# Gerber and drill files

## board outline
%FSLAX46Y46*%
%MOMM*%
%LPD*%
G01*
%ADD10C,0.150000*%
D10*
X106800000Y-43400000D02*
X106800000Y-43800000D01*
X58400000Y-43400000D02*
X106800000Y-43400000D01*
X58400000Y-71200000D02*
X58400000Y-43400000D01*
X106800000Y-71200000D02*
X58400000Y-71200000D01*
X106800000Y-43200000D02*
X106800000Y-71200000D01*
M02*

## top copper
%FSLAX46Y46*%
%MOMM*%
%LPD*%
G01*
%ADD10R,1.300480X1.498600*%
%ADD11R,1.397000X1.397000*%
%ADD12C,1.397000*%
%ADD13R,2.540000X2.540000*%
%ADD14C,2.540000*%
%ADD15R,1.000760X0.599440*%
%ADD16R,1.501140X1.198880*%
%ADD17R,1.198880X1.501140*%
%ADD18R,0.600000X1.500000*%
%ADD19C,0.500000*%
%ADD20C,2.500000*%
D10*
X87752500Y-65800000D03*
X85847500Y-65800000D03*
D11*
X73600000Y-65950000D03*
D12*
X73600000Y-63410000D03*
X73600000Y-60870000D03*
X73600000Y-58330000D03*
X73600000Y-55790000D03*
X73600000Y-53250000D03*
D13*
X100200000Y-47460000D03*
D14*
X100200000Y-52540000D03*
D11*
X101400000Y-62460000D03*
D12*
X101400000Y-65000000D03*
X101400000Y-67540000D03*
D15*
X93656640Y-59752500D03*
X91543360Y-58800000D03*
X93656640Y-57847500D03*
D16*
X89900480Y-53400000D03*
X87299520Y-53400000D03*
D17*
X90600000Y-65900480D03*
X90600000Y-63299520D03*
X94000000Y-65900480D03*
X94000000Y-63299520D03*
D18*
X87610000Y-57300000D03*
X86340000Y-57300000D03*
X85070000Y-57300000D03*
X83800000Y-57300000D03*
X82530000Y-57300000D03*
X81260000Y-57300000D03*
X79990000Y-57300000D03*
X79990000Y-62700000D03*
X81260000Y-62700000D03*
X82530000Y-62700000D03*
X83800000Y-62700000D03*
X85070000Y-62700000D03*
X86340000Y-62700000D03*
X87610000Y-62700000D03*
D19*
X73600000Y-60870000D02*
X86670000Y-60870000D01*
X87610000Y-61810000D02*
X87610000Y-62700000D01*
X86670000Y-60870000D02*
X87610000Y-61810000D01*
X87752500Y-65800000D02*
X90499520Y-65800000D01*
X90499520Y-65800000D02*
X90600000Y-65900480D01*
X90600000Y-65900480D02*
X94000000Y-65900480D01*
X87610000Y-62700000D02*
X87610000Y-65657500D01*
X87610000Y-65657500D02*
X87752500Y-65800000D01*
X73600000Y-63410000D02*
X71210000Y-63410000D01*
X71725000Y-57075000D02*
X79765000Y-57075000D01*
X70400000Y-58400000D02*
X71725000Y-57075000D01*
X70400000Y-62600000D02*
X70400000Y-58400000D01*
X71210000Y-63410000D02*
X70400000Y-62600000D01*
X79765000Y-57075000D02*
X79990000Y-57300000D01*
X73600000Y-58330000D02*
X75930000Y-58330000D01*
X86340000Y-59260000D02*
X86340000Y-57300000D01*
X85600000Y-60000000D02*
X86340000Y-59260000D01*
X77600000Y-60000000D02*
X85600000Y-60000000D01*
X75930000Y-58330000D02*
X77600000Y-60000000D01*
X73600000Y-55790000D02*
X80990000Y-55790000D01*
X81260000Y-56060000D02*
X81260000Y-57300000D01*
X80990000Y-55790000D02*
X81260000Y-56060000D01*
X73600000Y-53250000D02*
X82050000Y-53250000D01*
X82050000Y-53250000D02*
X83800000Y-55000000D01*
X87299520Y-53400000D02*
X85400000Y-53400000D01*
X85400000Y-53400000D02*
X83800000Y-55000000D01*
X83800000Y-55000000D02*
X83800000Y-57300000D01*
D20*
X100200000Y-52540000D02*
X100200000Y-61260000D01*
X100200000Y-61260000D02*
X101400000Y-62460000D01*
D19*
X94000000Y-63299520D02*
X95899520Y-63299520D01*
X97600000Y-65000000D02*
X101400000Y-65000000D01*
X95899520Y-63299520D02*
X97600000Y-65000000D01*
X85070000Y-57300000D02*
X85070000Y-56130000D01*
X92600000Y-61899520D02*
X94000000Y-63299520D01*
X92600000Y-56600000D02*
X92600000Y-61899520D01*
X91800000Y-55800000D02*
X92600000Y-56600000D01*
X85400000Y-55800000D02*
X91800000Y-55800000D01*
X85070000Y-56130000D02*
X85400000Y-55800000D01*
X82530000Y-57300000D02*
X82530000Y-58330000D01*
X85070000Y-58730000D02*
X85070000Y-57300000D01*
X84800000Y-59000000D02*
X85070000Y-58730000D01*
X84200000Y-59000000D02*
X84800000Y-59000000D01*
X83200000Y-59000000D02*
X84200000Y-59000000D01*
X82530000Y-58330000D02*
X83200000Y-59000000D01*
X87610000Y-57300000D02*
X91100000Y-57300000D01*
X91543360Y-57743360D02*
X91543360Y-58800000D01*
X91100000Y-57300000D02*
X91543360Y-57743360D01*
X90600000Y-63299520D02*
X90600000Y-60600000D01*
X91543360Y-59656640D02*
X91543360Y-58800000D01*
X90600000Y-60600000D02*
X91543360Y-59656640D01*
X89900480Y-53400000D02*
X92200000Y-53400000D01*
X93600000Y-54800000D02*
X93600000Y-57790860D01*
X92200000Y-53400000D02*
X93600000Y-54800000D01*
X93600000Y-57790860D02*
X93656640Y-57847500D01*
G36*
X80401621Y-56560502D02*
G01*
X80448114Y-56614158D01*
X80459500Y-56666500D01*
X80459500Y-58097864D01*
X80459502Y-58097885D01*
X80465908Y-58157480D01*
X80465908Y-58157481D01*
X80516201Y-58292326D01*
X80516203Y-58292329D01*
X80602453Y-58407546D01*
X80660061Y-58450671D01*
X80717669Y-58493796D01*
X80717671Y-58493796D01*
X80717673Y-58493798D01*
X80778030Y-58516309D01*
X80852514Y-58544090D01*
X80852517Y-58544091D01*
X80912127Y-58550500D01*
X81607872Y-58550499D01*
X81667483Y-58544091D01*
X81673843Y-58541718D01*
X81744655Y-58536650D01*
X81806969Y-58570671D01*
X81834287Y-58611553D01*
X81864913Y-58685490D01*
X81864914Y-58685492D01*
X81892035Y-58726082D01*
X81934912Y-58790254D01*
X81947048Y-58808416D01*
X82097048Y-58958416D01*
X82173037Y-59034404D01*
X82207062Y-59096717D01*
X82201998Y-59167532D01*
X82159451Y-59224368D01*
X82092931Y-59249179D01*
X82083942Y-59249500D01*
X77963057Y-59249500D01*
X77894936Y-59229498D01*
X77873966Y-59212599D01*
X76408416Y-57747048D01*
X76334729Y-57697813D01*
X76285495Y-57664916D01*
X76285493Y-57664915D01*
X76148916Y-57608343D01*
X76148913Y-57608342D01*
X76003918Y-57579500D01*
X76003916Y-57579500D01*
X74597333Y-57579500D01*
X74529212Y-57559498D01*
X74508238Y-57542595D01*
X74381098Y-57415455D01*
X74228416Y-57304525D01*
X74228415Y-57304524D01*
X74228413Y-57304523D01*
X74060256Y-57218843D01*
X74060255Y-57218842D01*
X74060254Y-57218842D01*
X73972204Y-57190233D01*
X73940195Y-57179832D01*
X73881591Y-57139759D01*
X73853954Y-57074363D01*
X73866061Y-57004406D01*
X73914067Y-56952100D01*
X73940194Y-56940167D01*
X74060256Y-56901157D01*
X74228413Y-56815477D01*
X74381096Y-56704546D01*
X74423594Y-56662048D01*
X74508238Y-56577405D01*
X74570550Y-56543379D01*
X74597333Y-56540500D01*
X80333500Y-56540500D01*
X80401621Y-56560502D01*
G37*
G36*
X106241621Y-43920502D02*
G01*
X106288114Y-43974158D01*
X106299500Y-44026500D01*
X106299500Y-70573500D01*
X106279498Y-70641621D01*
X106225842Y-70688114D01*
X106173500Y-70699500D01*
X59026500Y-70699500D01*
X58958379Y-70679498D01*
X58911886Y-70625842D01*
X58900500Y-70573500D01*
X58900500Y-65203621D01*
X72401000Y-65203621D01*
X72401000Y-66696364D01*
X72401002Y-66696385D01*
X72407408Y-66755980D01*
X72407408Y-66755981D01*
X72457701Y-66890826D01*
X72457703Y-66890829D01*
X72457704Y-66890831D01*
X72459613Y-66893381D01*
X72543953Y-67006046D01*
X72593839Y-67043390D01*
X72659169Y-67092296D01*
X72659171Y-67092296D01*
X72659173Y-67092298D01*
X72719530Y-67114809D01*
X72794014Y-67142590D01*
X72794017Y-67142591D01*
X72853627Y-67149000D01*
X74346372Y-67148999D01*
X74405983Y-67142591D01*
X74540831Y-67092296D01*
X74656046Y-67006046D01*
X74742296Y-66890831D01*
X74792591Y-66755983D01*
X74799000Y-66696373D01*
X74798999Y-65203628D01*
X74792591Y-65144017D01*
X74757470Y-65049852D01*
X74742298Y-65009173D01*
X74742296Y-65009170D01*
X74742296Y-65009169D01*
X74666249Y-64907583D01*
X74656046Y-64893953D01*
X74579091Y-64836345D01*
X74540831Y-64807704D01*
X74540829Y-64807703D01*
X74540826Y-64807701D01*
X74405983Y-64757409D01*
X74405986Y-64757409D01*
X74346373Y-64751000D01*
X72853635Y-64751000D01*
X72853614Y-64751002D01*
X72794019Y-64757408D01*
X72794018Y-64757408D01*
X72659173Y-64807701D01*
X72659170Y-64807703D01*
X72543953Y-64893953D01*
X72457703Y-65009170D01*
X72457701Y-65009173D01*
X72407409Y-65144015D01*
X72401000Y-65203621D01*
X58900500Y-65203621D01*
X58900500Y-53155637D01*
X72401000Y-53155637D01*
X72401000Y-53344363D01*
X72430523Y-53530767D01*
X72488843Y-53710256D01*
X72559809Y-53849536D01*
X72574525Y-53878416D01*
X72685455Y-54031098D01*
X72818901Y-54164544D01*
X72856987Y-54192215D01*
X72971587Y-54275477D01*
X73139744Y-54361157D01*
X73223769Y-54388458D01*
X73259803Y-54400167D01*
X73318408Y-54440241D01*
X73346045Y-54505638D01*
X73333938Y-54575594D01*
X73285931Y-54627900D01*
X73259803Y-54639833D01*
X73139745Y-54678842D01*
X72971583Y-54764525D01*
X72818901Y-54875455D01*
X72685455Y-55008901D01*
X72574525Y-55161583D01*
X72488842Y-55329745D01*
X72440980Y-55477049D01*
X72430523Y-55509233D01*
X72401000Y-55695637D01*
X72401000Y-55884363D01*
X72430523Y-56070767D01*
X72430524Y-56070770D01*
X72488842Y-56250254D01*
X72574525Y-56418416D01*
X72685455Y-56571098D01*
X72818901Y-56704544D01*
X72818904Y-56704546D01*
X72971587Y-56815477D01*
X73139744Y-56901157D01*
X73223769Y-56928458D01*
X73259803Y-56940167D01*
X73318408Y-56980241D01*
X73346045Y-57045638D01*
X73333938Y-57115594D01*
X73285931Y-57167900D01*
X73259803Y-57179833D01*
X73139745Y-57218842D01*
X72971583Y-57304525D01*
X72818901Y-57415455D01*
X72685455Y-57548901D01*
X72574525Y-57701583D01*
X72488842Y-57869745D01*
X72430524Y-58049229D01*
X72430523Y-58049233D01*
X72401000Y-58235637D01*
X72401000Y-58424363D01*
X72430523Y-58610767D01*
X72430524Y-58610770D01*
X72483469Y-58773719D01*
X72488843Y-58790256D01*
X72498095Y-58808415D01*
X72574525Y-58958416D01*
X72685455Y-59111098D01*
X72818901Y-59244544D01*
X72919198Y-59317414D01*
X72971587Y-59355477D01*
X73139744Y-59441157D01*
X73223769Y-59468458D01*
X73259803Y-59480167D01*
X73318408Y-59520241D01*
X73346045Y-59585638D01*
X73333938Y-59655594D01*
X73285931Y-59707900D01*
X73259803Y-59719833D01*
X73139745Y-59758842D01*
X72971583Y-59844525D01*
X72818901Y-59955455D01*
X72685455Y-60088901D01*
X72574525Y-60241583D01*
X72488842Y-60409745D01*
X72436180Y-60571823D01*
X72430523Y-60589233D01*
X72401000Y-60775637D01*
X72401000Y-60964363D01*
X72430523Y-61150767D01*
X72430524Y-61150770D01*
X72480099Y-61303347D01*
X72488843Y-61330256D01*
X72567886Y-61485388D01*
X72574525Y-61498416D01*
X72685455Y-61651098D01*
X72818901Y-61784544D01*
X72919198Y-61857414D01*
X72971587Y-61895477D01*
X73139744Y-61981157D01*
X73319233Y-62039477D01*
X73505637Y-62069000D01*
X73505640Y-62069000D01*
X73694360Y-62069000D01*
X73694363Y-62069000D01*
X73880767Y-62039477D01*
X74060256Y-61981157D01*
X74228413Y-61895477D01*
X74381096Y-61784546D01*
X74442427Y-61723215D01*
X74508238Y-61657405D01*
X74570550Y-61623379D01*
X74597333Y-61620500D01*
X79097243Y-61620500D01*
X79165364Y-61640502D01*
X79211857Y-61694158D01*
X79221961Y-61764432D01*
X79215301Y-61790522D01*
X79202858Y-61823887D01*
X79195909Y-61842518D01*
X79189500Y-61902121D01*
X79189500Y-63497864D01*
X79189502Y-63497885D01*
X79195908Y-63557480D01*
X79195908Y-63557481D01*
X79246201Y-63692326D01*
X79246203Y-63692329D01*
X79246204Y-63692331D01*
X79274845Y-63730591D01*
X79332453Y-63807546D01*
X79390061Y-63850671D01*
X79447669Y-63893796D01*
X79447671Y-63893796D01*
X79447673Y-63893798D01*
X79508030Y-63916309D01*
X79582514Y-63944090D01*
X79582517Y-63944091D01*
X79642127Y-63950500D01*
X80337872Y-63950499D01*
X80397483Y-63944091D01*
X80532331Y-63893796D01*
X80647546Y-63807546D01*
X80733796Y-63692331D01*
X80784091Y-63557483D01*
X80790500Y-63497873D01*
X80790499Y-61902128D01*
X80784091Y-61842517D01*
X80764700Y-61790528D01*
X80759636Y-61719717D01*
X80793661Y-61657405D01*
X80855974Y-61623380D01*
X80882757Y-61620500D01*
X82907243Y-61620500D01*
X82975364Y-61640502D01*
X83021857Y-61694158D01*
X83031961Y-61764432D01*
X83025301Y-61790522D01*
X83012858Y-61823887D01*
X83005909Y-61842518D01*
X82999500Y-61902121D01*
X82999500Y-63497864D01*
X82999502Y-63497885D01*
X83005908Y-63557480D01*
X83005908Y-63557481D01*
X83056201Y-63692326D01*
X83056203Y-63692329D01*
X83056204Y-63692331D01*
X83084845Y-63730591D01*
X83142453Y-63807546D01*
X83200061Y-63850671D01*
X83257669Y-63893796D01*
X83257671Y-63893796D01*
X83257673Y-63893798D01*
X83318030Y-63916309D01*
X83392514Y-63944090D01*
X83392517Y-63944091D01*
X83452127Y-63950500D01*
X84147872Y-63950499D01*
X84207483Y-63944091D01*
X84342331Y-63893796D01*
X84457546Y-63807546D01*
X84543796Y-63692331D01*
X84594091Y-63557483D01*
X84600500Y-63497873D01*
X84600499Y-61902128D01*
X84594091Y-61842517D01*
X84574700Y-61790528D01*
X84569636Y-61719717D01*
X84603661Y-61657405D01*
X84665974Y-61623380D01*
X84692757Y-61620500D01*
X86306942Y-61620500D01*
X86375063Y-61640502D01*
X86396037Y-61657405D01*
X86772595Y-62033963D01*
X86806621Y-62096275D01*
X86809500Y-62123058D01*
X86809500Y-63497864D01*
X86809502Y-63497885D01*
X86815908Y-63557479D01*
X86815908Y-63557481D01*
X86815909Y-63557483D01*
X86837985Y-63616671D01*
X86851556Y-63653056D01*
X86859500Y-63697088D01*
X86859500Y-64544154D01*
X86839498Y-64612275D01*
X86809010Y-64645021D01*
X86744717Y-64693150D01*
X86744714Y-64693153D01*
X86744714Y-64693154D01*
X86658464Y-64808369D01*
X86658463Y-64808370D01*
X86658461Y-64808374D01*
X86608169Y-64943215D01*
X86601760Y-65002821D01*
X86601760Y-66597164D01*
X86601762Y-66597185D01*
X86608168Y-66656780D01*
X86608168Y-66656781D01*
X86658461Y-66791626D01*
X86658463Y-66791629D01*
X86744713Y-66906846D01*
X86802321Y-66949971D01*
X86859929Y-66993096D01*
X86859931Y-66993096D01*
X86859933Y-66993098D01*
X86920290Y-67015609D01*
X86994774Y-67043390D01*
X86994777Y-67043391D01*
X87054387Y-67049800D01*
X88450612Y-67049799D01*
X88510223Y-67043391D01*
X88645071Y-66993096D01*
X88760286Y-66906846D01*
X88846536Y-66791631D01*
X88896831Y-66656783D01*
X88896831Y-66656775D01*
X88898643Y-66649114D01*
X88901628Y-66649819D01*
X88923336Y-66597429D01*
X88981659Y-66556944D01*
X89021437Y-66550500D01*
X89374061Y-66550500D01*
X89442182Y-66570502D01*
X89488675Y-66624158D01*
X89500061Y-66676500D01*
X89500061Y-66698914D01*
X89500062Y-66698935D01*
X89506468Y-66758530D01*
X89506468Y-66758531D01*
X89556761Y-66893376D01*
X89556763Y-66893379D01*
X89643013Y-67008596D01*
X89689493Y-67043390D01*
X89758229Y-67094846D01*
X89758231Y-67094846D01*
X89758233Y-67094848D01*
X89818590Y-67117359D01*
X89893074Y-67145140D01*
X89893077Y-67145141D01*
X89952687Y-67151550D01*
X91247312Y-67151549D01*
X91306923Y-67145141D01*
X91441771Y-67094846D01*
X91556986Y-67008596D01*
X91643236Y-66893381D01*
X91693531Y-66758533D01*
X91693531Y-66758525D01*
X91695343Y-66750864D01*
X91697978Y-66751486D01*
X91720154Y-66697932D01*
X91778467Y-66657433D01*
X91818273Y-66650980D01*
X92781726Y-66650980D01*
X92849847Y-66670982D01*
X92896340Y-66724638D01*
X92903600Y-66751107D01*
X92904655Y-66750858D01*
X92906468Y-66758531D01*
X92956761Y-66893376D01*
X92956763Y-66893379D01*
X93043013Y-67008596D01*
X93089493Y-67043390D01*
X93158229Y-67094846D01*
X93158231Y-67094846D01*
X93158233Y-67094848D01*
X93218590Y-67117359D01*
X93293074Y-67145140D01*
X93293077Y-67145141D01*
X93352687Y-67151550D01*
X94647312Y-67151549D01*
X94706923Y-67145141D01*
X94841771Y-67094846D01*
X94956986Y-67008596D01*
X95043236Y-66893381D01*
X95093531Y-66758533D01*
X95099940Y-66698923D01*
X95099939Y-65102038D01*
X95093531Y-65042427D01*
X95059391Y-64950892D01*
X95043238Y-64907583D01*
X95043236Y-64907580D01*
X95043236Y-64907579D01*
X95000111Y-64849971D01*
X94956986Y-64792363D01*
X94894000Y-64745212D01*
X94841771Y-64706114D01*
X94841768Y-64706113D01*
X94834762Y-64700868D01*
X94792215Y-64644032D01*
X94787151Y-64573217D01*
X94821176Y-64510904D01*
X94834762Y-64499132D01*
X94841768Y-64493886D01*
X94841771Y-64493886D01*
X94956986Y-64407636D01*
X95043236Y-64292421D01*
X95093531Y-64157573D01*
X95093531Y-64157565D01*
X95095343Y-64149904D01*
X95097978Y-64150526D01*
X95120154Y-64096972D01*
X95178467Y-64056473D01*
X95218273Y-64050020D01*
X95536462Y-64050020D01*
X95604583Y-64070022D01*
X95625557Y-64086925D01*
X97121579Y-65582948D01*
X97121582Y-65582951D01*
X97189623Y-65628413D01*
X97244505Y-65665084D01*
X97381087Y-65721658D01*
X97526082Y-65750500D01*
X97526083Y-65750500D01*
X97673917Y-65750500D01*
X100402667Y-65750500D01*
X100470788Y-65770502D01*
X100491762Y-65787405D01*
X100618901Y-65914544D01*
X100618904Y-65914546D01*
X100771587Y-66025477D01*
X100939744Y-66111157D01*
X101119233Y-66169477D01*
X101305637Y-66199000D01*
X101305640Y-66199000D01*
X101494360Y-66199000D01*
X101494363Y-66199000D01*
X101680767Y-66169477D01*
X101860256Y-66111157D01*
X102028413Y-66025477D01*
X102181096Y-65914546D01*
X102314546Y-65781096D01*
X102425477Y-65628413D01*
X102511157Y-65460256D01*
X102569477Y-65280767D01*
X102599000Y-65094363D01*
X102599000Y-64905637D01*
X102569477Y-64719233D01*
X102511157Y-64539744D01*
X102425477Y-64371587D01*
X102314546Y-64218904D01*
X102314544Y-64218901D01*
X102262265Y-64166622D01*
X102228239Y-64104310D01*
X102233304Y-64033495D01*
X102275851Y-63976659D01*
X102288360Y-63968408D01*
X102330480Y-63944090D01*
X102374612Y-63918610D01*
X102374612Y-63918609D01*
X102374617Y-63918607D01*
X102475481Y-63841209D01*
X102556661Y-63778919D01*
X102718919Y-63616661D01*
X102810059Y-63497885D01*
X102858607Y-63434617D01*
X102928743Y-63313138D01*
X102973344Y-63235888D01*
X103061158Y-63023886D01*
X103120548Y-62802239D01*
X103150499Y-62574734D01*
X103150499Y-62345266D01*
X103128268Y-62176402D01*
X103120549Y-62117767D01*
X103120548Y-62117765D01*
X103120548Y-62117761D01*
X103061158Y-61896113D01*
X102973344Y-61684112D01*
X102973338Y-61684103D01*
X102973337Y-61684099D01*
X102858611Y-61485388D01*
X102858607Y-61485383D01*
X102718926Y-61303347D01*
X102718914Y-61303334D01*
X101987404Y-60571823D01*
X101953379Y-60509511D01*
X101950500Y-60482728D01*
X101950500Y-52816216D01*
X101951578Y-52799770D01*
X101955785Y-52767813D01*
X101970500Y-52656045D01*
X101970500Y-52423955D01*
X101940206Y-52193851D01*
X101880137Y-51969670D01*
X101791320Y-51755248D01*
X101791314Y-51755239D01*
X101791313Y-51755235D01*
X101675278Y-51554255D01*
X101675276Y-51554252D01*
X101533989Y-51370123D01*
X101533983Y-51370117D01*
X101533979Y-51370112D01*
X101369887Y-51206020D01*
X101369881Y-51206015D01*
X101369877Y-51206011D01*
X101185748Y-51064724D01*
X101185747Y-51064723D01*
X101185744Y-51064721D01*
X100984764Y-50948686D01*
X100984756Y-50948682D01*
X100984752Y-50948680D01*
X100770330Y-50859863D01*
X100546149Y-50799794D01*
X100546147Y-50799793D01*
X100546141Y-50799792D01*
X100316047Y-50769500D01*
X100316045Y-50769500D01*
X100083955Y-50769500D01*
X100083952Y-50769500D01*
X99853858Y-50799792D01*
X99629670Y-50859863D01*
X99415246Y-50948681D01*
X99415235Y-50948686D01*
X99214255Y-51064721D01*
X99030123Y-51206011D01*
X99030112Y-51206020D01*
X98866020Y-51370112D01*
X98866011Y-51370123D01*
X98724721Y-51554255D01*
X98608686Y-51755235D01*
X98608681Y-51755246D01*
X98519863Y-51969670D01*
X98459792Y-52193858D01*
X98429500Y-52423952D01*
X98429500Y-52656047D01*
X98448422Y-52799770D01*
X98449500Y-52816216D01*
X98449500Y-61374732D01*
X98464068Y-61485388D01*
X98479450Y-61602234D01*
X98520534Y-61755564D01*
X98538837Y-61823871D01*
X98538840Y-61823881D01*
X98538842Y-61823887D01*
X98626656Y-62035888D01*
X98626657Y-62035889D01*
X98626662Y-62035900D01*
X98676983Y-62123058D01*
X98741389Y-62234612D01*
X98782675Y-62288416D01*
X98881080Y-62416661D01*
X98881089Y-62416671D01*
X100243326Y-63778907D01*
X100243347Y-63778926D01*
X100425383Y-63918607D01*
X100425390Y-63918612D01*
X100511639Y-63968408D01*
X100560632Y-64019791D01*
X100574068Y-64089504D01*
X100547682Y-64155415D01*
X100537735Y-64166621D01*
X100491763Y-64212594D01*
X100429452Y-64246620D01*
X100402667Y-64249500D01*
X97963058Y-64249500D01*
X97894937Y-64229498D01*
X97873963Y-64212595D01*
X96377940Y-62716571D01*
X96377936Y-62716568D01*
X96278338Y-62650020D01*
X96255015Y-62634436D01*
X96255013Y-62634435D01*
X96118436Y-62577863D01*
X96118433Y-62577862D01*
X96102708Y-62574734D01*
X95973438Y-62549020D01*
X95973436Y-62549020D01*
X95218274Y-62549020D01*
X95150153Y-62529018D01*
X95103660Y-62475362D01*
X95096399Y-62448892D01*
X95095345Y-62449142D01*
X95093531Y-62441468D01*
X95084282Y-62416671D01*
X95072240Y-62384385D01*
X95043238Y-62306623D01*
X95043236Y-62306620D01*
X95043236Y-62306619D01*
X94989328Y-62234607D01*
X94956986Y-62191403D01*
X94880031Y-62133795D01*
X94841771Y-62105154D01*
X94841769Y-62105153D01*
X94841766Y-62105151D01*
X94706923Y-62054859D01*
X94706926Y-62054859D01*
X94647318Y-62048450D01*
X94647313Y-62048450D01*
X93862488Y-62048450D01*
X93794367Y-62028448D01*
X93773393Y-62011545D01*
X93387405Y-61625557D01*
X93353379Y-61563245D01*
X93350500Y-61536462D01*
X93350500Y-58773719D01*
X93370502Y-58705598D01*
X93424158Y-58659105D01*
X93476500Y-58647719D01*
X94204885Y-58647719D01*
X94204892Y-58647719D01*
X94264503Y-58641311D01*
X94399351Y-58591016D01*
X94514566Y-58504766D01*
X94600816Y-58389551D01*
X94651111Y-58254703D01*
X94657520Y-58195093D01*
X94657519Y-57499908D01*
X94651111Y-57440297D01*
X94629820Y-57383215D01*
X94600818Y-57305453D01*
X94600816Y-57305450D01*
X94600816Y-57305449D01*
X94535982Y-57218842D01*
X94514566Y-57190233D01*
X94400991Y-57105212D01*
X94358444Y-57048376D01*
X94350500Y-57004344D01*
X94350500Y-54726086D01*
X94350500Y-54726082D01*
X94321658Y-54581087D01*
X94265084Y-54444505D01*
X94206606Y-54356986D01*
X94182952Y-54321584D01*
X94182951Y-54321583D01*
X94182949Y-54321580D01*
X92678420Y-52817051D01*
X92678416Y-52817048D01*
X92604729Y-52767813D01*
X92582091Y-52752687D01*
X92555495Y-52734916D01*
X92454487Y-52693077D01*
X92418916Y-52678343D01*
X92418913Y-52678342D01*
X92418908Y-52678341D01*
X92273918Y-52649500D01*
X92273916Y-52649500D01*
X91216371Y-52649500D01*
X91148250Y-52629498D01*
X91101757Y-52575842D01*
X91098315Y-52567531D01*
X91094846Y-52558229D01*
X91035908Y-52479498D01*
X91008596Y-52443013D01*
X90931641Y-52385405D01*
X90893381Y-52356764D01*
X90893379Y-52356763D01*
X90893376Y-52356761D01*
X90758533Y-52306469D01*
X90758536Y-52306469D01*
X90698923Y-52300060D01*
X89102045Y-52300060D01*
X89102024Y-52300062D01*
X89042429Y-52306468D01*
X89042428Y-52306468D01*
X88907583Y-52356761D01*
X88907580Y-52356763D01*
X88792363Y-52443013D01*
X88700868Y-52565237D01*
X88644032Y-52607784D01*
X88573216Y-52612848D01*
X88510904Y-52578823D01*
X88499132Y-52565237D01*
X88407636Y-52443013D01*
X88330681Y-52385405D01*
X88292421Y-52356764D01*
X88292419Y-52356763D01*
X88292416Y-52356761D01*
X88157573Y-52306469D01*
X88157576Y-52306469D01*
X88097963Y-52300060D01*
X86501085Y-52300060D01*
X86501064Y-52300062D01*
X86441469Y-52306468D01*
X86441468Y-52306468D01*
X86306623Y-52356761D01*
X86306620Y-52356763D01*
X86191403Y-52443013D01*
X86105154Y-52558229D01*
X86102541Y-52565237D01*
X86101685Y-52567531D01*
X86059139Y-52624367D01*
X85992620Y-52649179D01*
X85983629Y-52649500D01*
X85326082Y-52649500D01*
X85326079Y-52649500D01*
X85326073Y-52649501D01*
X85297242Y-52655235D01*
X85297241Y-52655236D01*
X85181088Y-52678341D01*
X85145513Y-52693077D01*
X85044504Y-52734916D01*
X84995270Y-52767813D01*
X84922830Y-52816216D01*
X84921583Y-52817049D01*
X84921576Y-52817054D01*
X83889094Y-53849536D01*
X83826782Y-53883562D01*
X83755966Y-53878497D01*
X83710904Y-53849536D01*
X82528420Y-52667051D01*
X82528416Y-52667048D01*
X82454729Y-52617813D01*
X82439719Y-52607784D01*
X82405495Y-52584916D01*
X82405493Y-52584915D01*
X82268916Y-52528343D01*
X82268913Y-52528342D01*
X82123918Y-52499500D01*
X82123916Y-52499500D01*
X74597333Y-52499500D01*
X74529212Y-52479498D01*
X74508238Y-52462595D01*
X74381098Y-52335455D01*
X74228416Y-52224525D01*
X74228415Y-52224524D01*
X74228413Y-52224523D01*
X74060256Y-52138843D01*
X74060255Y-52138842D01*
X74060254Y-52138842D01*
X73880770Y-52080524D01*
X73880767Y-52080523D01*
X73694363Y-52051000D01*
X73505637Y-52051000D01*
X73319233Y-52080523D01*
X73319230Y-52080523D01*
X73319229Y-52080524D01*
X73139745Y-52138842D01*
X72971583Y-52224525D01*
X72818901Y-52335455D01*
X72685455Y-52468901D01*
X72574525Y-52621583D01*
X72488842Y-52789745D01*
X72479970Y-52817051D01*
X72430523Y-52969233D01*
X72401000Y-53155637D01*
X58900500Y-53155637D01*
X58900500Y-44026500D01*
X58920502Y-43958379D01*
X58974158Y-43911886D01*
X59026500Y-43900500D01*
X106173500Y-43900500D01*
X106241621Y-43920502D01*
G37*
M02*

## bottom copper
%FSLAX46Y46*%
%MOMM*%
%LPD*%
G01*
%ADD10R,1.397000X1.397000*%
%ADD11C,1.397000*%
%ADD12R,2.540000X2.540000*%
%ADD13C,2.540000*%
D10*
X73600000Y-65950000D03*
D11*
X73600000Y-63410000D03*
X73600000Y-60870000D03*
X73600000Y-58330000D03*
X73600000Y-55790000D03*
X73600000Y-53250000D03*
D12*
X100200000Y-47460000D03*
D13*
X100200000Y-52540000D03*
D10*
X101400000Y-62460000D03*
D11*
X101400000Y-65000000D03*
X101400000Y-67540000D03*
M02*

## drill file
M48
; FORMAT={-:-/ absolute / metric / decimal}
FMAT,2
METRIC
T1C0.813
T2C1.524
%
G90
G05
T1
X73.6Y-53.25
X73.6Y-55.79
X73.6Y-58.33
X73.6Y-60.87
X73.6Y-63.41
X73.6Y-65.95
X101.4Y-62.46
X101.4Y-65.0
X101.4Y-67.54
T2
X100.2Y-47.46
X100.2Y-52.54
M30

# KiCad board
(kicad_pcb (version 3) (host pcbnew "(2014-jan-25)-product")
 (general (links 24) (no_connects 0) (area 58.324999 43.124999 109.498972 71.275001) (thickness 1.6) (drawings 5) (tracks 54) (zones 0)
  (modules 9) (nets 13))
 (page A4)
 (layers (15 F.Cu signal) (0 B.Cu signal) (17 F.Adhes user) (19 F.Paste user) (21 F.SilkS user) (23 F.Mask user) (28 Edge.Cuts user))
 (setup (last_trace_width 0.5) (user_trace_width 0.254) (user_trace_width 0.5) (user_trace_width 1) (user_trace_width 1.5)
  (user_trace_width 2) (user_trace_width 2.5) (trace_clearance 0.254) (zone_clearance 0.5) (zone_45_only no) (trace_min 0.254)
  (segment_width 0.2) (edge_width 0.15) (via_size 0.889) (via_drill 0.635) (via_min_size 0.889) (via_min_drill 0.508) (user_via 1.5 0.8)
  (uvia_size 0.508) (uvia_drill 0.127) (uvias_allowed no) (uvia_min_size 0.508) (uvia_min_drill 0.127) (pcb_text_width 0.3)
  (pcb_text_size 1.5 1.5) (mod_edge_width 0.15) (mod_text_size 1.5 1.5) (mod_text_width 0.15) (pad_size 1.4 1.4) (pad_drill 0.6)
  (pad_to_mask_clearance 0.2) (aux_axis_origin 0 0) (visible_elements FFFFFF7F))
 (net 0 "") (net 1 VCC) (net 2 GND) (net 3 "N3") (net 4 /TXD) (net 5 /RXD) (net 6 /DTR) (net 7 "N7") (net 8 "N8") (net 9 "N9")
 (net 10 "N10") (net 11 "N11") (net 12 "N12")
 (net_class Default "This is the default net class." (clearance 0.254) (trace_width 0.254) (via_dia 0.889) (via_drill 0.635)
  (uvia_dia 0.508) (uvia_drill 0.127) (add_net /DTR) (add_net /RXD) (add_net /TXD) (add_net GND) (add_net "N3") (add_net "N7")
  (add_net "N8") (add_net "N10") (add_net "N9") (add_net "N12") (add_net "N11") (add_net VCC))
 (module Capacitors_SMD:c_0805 (layer F.Cu) (at 86.8 65.8)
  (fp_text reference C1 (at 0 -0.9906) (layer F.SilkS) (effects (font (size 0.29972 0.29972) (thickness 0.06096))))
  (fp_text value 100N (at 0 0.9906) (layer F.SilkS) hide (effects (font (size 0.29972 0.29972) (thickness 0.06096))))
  (pad 1 smd rect (at 0.9525 0) (size 1.30048 1.4986) (layers F.Cu F.Paste F.Mask) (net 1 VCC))
  (pad 2 smd rect (at -0.9525 0) (size 1.30048 1.4986) (layers F.Cu F.Paste F.Mask) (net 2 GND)))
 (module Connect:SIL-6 (layer F.Cu) (at 73.6 59.6 90)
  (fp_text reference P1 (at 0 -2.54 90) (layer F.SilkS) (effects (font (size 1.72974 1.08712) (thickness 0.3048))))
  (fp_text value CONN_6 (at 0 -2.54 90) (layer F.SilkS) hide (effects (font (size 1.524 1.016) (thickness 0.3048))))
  (pad 1 thru_hole rect (at -6.35 0 90) (size 1.397 1.397) (drill 0.8128) (layers *.Cu *.Mask F.SilkS) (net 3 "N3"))
  (pad 2 thru_hole circle (at -3.81 0 90) (size 1.397 1.397) (drill 0.8128) (layers *.Cu *.Mask F.SilkS) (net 2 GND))
  (pad 3 thru_hole circle (at -1.27 0 90) (size 1.397 1.397) (drill 0.8128) (layers *.Cu *.Mask F.SilkS) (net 1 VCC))
  (pad 4 thru_hole circle (at 1.27 0 90) (size 1.397 1.397) (drill 0.8128) (layers *.Cu *.Mask F.SilkS) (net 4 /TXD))
  (pad 5 thru_hole circle (at 3.81 0 90) (size 1.397 1.397) (drill 0.8128) (layers *.Cu *.Mask F.SilkS) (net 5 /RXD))
  (pad 6 thru_hole circle (at 6.35 0 90) (size 1.397 1.397) (drill 0.8128) (layers *.Cu *.Mask F.SilkS) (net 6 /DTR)))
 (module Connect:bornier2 (layer F.Cu) (at 100.2 50 270)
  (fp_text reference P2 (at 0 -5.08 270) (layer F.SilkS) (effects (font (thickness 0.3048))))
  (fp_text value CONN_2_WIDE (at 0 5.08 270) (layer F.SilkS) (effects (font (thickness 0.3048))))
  (pad 1 thru_hole rect (at -2.54 0 270) (size 2.54 2.54) (drill 1.524) (layers *.Cu *.Mask F.SilkS) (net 2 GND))
  (pad 2 thru_hole circle (at 2.54 0 270) (size 2.54 2.54) (drill 1.524) (layers *.Cu *.Mask F.SilkS) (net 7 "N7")))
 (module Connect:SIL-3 (layer F.Cu) (at 101.4 65 270)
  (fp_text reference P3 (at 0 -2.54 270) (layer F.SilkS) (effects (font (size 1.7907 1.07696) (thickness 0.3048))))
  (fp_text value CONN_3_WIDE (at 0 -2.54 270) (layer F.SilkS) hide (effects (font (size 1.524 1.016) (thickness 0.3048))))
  (pad 1 thru_hole rect (at -2.54 0 270) (size 1.397 1.397) (drill 0.8128) (layers *.Cu *.Mask F.SilkS) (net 7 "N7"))
  (pad 2 thru_hole circle (at 0 0 270) (size 1.397 1.397) (drill 0.8128) (layers *.Cu *.Mask F.SilkS) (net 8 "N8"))
  (pad 3 thru_hole circle (at 2.54 0 270) (size 1.397 1.397) (drill 0.8128) (layers *.Cu *.Mask F.SilkS) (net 2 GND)))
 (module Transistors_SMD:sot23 (layer F.Cu) (at 92.6 58.8 90)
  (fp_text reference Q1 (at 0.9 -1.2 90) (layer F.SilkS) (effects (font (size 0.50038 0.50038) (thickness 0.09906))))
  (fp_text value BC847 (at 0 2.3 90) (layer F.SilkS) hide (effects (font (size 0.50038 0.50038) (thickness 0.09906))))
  (pad 1 smd rect (at -0.9525 1.05664 90) (size 0.59944 1.00076) (layers F.Cu F.Paste F.Mask) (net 2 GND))
  (pad 3 smd rect (at 0 -1.05664 90) (size 0.59944 1.00076) (layers F.Cu F.Paste F.Mask) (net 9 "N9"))
  (pad 2 smd rect (at 0.9525 1.05664 90) (size 0.59944 1.00076) (layers F.Cu F.Paste F.Mask) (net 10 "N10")))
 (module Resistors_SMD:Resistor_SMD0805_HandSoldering (layer F.Cu) (at 88.6 53.4 180)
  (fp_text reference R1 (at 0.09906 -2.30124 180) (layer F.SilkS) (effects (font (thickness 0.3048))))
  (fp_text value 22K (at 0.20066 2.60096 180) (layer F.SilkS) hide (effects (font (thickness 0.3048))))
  (pad 1 smd rect (at -1.30048 0 180) (size 1.50114 1.19888) (layers F.Cu F.Paste F.Mask) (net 10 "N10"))
  (pad 2 smd rect (at 1.30048 0 180) (size 1.50114 1.19888) (layers F.Cu F.Paste F.Mask) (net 6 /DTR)))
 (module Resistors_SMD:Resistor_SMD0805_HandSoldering (layer F.Cu) (at 90.6 64.6 90)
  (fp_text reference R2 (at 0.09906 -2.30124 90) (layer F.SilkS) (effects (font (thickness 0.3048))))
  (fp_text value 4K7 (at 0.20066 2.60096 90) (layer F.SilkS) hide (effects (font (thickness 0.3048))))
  (pad 1 smd rect (at -1.30048 0 90) (size 1.50114 1.19888) (layers F.Cu F.Paste F.Mask) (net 1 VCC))
  (pad 2 smd rect (at 1.30048 0 90) (size 1.50114 1.19888) (layers F.Cu F.Paste F.Mask) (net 9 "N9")))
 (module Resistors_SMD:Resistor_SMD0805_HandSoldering (layer F.Cu) (at 94 64.6 90)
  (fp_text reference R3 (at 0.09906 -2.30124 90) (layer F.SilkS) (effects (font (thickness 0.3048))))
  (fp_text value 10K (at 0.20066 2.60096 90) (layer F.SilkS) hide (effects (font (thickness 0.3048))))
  (pad 1 smd rect (at -1.30048 0 90) (size 1.50114 1.19888) (layers F.Cu F.Paste F.Mask) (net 1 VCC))
  (pad 2 smd rect (at 1.30048 0 90) (size 1.50114 1.19888) (layers F.Cu F.Paste F.Mask) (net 8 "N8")))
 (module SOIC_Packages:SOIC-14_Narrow (layer F.Cu) (at 83.8 60 180)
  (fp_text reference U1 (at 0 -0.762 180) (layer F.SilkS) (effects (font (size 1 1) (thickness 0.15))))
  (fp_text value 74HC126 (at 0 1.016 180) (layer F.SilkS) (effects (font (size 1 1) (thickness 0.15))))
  (pad 1 smd rect (at -3.81 2.7 180) (size 0.6 1.5) (layers F.Cu F.Paste F.Mask) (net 9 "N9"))
  (pad 2 smd rect (at -2.54 2.7 180) (size 0.6 1.5) (layers F.Cu F.Paste F.Mask) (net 4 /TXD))
  (pad 3 smd rect (at -1.27 2.7 180) (size 0.6 1.5) (layers F.Cu F.Paste F.Mask) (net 8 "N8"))
  (pad 4 smd rect (at 0 2.7 180) (size 0.6 1.5) (layers F.Cu F.Paste F.Mask) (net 6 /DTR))
  (pad 5 smd rect (at 1.27 2.7 180) (size 0.6 1.5) (layers F.Cu F.Paste F.Mask) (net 8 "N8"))
  (pad 6 smd rect (at 2.54 2.7 180) (size 0.6 1.5) (layers F.Cu F.Paste F.Mask) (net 5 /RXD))
  (pad 7 smd rect (at 3.81 2.7 180) (size 0.6 1.5) (layers F.Cu F.Paste F.Mask) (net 2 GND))
  (pad 8 smd rect (at 3.81 -2.7 180) (size 0.6 1.5) (layers F.Cu F.Paste F.Mask) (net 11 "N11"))
  (pad 9 smd rect (at 2.54 -2.7 180) (size 0.6 1.5) (layers F.Cu F.Paste F.Mask) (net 2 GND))
  (pad 10 smd rect (at 1.27 -2.7 180) (size 0.6 1.5) (layers F.Cu F.Paste F.Mask) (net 2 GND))
  (pad 11 smd rect (at 0 -2.7 180) (size 0.6 1.5) (layers F.Cu F.Paste F.Mask) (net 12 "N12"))
  (pad 12 smd rect (at -1.27 -2.7 180) (size 0.6 1.5) (layers F.Cu F.Paste F.Mask) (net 2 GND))
  (pad 13 smd rect (at -2.54 -2.7 180) (size 0.6 1.5) (layers F.Cu F.Paste F.Mask) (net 2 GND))
  (pad 14 smd rect (at -3.81 -2.7 180) (size 0.6 1.5) (layers F.Cu F.Paste F.Mask) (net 1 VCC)))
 (gr_line (start 106.8 43.4) (end 106.8 43.8) (angle 90) (layer Edge.Cuts) (width 0.15))
 (gr_line (start 58.4 43.4) (end 106.8 43.4) (angle 90) (layer Edge.Cuts) (width 0.15))
 (gr_line (start 58.4 71.2) (end 58.4 43.4) (angle 90) (layer Edge.Cuts) (width 0.15))
 (gr_line (start 106.8 71.2) (end 58.4 71.2) (angle 90) (layer Edge.Cuts) (width 0.15))
 (gr_line (start 106.8 43.2) (end 106.8 71.2) (angle 90) (layer Edge.Cuts) (width 0.15))
 (segment (start 73.6 60.87) (end 86.67 60.87) (width 0.5) (layer F.Cu) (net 1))
 (segment (start 87.61 61.81) (end 87.61 62.7) (width 0.5) (layer F.Cu) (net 1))
 (segment (start 86.67 60.87) (end 87.61 61.81) (width 0.5) (layer F.Cu) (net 1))
 (segment (start 87.7525 65.8) (end 90.49952 65.8) (width 0.5) (layer F.Cu) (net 1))
 (segment (start 90.49952 65.8) (end 90.6 65.90048) (width 0.5) (layer F.Cu) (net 1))
 (segment (start 90.6 65.90048) (end 94 65.90048) (width 0.5) (layer F.Cu) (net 1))
 (segment (start 87.61 62.7) (end 87.61 65.6575) (width 0.5) (layer F.Cu) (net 1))
 (segment (start 87.61 65.6575) (end 87.7525 65.8) (width 0.5) (layer F.Cu) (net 1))
 (segment (start 73.6 63.41) (end 71.21 63.41) (width 0.5) (layer F.Cu) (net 2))
 (segment (start 71.725 57.075) (end 79.765 57.075) (width 0.5) (layer F.Cu) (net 2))
 (segment (start 70.4 58.4) (end 71.725 57.075) (width 0.5) (layer F.Cu) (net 2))
 (segment (start 70.4 62.6) (end 70.4 58.4) (width 0.5) (layer F.Cu) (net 2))
 (segment (start 71.21 63.41) (end 70.4 62.6) (width 0.5) (layer F.Cu) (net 2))
 (segment (start 79.765 57.075) (end 79.99 57.3) (width 0.5) (layer F.Cu) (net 2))
 (segment (start 73.6 58.33) (end 75.93 58.33) (width 0.5) (layer F.Cu) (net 4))
 (segment (start 86.34 59.26) (end 86.34 57.3) (width 0.5) (layer F.Cu) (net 4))
 (segment (start 85.6 60) (end 86.34 59.26) (width 0.5) (layer F.Cu) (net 4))
 (segment (start 77.6 60) (end 85.6 60) (width 0.5) (layer F.Cu) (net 4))
 (segment (start 75.93 58.33) (end 77.6 60) (width 0.5) (layer F.Cu) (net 4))
 (segment (start 73.6 55.79) (end 80.99 55.79) (width 0.5) (layer F.Cu) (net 5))
 (segment (start 81.26 56.06) (end 81.26 57.3) (width 0.5) (layer F.Cu) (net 5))
 (segment (start 80.99 55.79) (end 81.26 56.06) (width 0.5) (layer F.Cu) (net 5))
 (segment (start 73.6 53.25) (end 82.05 53.25) (width 0.5) (layer F.Cu) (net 6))
 (segment (start 82.05 53.25) (end 83.8 55) (width 0.5) (layer F.Cu) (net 6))
 (segment (start 87.29952 53.4) (end 85.4 53.4) (width 0.5) (layer F.Cu) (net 6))
 (segment (start 85.4 53.4) (end 83.8 55) (width 0.5) (layer F.Cu) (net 6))
 (segment (start 83.8 55) (end 83.8 57.3) (width 0.5) (layer F.Cu) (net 6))
 (segment (start 100.2 52.54) (end 100.2 61.26) (width 2.5) (layer F.Cu) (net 7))
 (segment (start 100.2 61.26) (end 101.4 62.46) (width 2.5) (layer F.Cu) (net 7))
 (segment (start 94 63.29952) (end 95.89952 63.29952) (width 0.5) (layer F.Cu) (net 8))
 (segment (start 97.6 65) (end 101.4 65) (width 0.5) (layer F.Cu) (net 8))
 (segment (start 95.89952 63.29952) (end 97.6 65) (width 0.5) (layer F.Cu) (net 8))
 (segment (start 85.07 57.3) (end 85.07 56.13) (width 0.5) (layer F.Cu) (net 8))
 (segment (start 92.6 61.89952) (end 94 63.29952) (width 0.5) (layer F.Cu) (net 8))
 (segment (start 92.6 56.6) (end 92.6 61.89952) (width 0.5) (layer F.Cu) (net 8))
 (segment (start 91.8 55.8) (end 92.6 56.6) (width 0.5) (layer F.Cu) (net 8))
 (segment (start 85.4 55.8) (end 91.8 55.8) (width 0.5) (layer F.Cu) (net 8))
 (segment (start 85.07 56.13) (end 85.4 55.8) (width 0.5) (layer F.Cu) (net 8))
 (segment (start 82.53 57.3) (end 82.53 58.33) (width 0.5) (layer F.Cu) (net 8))
 (segment (start 85.07 58.73) (end 85.07 57.3) (width 0.5) (layer F.Cu) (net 8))
 (segment (start 84.8 59) (end 85.07 58.73) (width 0.5) (layer F.Cu) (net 8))
 (segment (start 84.2 59) (end 84.8 59) (width 0.5) (layer F.Cu) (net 8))
 (segment (start 83.2 59) (end 84.2 59) (width 0.5) (layer F.Cu) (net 8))
 (segment (start 82.53 58.33) (end 83.2 59) (width 0.5) (layer F.Cu) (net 8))
 (segment (start 87.61 57.3) (end 91.1 57.3) (width 0.5) (layer F.Cu) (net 9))
 (segment (start 91.54336 57.74336) (end 91.54336 58.8) (width 0.5) (layer F.Cu) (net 9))
 (segment (start 91.1 57.3) (end 91.54336 57.74336) (width 0.5) (layer F.Cu) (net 9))
 (segment (start 90.6 63.29952) (end 90.6 60.6) (width 0.5) (layer F.Cu) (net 9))
 (segment (start 91.54336 59.65664) (end 91.54336 58.8) (width 0.5) (layer F.Cu) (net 9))
 (segment (start 90.6 60.6) (end 91.54336 59.65664) (width 0.5) (layer F.Cu) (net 9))
 (segment (start 89.90048 53.4) (end 92.2 53.4) (width 0.5) (layer F.Cu) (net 10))
 (segment (start 93.6 54.8) (end 93.6 57.79086) (width 0.5) (layer F.Cu) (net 10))
 (segment (start 92.2 53.4) (end 93.6 54.8) (width 0.5) (layer F.Cu) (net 10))
 (segment (start 93.6 57.79086) (end 93.65664 57.8475) (width 0.5) (layer F.Cu) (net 10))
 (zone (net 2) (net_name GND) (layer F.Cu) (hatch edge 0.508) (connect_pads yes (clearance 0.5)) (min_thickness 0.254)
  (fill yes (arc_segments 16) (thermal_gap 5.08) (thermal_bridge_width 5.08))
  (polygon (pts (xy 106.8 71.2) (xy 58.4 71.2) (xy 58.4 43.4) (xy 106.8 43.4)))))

